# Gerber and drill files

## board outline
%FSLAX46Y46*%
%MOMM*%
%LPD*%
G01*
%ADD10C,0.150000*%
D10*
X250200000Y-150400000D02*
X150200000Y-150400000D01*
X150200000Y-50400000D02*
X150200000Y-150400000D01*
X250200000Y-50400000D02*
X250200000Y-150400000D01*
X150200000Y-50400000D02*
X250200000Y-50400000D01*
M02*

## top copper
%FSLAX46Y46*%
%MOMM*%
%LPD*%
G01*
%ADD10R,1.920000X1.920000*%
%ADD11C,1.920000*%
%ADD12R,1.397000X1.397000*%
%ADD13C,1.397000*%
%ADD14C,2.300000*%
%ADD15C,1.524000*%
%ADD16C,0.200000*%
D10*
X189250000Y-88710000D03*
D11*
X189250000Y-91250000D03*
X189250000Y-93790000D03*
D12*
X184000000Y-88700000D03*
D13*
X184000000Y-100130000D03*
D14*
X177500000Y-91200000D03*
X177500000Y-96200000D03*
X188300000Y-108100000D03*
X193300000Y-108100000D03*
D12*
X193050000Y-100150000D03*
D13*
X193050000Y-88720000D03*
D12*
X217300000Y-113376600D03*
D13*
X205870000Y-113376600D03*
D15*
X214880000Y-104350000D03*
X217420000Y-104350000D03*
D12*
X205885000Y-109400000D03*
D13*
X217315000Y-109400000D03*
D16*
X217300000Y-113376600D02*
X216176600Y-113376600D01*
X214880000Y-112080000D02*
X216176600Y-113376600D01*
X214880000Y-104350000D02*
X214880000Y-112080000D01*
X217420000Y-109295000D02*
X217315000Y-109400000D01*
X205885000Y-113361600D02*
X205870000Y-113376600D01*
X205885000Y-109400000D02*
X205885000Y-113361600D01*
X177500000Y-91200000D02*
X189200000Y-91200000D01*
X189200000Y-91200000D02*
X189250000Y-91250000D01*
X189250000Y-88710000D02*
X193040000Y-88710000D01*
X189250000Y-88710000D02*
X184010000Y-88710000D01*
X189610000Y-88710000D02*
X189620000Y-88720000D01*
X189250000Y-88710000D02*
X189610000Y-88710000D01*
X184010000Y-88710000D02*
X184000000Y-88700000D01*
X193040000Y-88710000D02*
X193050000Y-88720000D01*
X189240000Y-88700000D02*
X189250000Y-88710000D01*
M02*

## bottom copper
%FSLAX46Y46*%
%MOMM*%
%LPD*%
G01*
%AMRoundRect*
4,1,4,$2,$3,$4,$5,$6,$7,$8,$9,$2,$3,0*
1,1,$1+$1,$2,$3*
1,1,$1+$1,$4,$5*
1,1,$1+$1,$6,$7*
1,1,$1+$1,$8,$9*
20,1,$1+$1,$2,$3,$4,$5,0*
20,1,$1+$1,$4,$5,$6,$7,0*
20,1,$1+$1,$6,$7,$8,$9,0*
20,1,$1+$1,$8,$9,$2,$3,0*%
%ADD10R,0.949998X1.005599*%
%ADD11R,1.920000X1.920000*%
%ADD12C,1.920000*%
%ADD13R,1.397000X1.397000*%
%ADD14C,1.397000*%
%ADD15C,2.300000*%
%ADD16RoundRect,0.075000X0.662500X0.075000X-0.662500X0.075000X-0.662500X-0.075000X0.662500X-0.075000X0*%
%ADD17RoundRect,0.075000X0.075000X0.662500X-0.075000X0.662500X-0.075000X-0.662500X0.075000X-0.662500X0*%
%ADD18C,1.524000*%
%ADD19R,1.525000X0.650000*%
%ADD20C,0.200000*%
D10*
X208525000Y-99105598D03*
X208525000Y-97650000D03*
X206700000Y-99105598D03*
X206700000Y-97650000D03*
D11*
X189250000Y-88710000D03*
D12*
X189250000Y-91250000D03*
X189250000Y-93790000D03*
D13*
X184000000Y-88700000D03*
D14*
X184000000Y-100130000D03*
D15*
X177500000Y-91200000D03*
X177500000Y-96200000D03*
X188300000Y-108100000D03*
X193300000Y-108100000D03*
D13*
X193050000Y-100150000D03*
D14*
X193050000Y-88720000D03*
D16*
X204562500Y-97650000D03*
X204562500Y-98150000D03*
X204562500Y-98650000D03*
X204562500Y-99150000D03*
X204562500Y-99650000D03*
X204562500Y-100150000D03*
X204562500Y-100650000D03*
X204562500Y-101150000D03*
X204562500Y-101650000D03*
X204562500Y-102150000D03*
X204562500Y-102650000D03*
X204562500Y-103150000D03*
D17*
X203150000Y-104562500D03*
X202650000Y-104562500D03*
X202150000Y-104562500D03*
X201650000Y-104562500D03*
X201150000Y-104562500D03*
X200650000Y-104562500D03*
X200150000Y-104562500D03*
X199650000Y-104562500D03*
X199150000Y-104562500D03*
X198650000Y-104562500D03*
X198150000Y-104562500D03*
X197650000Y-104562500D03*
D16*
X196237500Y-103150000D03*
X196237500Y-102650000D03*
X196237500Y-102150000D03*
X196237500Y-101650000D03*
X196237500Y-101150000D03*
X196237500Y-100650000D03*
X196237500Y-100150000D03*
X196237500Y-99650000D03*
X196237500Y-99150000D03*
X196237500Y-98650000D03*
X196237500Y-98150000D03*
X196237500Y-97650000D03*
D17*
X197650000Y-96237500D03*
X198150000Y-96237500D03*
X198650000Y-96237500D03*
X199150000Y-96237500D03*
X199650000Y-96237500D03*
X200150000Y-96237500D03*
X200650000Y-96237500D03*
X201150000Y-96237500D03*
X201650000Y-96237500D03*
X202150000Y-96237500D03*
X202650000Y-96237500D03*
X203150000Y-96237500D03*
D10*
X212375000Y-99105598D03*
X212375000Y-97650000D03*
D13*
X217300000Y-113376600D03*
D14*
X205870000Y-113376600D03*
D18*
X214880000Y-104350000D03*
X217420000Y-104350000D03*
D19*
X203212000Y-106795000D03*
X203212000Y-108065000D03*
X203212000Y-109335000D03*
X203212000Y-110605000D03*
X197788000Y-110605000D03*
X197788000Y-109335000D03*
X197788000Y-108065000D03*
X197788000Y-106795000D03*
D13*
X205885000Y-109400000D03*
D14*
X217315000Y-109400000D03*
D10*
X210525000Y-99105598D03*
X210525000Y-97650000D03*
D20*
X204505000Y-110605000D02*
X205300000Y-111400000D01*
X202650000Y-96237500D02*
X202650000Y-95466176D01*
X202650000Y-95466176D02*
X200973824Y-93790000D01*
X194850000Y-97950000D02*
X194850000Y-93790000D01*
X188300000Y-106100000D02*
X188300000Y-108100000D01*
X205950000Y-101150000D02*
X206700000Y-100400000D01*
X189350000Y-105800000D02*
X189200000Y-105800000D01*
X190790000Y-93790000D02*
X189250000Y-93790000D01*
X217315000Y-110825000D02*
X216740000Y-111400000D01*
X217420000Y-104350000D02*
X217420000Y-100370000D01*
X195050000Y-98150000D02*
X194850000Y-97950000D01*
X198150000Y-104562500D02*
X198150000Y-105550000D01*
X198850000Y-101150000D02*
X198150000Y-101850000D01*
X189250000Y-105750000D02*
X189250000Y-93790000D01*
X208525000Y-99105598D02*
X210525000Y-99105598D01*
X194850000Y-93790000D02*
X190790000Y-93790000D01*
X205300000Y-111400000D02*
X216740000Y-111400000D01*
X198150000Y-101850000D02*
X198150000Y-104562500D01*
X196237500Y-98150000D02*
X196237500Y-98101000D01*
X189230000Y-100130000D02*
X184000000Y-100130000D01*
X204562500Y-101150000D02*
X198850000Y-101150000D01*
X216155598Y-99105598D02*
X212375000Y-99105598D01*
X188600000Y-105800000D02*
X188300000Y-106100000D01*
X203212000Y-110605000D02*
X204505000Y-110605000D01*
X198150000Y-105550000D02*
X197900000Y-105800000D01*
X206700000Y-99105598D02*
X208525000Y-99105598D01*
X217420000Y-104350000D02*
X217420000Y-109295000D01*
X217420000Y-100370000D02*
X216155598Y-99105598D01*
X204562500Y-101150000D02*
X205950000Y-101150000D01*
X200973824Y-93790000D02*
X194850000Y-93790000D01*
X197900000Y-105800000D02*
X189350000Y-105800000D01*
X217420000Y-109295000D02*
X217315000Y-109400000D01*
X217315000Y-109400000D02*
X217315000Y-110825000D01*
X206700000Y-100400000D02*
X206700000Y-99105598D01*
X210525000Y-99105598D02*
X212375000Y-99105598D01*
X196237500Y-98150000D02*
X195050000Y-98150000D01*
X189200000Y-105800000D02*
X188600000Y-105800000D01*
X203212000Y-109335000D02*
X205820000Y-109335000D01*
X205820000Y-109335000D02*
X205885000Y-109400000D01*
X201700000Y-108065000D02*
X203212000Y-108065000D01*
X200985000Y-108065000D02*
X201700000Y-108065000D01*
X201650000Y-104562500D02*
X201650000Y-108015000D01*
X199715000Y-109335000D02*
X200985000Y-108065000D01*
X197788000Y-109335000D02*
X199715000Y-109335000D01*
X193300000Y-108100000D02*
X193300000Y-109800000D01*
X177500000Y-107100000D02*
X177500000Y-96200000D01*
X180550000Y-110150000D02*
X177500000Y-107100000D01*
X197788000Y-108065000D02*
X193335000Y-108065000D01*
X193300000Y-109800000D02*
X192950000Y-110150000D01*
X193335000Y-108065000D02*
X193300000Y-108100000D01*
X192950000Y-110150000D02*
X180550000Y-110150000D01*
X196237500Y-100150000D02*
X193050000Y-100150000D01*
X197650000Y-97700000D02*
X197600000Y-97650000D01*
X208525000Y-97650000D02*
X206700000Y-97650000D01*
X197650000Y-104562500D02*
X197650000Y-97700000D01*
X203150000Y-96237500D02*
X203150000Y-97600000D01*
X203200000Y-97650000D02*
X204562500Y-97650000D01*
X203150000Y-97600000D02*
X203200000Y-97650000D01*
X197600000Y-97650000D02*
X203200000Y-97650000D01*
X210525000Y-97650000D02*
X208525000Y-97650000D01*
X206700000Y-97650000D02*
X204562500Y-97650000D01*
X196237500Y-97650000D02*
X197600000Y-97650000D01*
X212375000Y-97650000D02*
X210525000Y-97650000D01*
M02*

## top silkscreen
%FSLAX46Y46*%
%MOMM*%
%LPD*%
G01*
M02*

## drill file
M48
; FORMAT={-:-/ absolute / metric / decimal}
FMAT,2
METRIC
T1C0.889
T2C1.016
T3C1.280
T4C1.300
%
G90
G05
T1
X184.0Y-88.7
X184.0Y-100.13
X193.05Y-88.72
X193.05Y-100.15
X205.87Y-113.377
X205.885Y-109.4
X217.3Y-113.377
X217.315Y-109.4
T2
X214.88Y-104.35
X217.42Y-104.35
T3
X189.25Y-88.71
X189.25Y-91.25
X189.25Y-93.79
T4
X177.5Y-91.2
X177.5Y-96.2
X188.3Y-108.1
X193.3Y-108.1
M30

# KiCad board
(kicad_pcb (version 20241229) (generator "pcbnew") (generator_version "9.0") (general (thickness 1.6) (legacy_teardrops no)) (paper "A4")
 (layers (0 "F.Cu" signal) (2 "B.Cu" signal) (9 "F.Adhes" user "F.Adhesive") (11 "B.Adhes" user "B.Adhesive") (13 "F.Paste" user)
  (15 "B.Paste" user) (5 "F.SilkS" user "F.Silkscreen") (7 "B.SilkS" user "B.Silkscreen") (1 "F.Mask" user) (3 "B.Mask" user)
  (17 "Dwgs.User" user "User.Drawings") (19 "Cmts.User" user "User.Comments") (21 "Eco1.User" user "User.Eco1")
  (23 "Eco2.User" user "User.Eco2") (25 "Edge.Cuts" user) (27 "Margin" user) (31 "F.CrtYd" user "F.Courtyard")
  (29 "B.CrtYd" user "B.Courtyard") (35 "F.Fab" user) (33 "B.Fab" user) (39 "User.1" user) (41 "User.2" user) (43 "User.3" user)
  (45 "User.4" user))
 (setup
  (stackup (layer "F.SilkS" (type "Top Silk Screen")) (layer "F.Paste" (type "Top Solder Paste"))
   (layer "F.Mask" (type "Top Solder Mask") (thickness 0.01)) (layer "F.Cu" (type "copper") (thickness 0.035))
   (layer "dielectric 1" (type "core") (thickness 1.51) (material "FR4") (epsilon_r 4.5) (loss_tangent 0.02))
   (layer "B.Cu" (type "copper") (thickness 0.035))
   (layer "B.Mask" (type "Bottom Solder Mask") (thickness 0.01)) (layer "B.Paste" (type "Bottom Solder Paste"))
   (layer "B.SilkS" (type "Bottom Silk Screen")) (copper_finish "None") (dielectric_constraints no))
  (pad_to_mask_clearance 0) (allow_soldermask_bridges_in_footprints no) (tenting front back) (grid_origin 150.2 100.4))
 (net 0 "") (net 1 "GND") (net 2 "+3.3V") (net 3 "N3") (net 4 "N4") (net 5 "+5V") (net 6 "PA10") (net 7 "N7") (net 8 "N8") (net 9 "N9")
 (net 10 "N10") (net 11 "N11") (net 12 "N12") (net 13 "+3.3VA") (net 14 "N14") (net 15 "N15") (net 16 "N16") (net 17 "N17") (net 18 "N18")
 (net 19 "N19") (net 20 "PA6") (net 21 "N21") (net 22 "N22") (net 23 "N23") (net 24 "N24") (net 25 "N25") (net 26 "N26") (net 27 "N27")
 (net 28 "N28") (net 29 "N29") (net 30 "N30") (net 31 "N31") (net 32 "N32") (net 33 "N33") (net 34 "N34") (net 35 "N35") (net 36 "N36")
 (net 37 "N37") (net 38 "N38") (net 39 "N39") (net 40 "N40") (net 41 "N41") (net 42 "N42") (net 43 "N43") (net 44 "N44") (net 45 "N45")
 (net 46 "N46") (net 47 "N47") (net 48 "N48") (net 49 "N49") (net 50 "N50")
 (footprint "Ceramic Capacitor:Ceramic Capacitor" (layer "B.Cu") (at 208.525 98.377799 90)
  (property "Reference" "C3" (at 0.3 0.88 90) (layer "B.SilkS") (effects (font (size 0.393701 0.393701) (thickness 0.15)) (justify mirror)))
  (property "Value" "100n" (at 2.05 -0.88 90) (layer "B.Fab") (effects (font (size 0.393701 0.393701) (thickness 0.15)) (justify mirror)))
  (pad "1" smd rect (at -0.727799 0 90) (size 1.005599 0.949998) (layers "B.Cu" "B.Mask" "B.Paste") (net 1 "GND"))
  (pad "2" smd rect (at 0.727799 0 90) (size 1.005599 0.949998) (layers "B.Cu" "B.Mask" "B.Paste") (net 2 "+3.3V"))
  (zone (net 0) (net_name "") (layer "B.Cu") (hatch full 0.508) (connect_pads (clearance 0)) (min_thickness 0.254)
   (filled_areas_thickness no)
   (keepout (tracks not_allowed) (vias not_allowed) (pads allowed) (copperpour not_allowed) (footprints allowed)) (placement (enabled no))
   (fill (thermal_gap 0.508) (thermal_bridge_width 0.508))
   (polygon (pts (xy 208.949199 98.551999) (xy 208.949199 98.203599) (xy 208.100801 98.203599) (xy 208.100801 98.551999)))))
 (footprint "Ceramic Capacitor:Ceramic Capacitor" (layer "B.Cu") (at 206.7 98.377799 90)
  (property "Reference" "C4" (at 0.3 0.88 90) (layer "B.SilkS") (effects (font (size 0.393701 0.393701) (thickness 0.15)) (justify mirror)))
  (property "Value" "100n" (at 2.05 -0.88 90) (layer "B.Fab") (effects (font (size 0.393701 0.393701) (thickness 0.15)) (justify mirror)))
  (pad "1" smd rect (at -0.727799 0 90) (size 1.005599 0.949998) (layers "B.Cu" "B.Mask" "B.Paste") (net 1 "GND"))
  (pad "2" smd rect (at 0.727799 0 90) (size 1.005599 0.949998) (layers "B.Cu" "B.Mask" "B.Paste") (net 2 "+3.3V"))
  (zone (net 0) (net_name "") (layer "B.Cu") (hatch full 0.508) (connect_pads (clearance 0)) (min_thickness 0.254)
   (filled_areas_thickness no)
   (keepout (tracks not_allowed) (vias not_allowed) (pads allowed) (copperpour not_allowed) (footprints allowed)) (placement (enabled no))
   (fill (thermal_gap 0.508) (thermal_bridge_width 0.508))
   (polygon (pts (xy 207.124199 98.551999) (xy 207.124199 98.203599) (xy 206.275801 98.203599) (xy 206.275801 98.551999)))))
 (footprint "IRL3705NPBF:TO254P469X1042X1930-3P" (layer "B.Cu") (at 189.25 88.71 -90)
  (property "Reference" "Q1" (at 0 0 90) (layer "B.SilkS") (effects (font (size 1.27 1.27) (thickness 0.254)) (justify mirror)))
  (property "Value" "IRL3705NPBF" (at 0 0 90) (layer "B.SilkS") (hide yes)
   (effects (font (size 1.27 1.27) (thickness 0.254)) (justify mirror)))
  (pad "1" thru_hole rect (at 0 0 270) (size 1.92 1.92) (drill 1.28) (layers "*.Cu" "*.Mask") (remove_unused_layers no) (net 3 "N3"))
  (pad "2" thru_hole circle (at 2.54 0 270) (size 1.92 1.92) (drill 1.28) (layers "*.Cu" "*.Mask") (remove_unused_layers no) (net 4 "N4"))
  (pad "3" thru_hole circle (at 5.08 0 270) (size 1.92 1.92) (drill 1.28) (layers "*.Cu" "*.Mask") (remove_unused_layers no) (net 1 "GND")))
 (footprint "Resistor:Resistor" (layer "B.Cu") (at 184 88.7 -90)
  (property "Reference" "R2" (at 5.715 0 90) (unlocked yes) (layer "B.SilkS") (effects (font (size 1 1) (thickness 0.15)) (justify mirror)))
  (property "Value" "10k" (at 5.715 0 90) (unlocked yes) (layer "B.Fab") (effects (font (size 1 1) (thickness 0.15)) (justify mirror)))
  (pad "1" thru_hole rect (at 0 0 270) (size 1.397 1.397) (drill 0.889) (layers "*.Cu" "*.Mask") (remove_unused_layers no) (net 3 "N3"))
  (pad "2" thru_hole circle (at 11.43 0 270) (size 1.397 1.397) (drill 0.889) (layers "*.Cu" "*.Mask") (remove_unused_layers no)
   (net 1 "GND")))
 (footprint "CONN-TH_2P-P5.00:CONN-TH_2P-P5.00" (layer "B.Cu") (at 181.75 88.7 -90)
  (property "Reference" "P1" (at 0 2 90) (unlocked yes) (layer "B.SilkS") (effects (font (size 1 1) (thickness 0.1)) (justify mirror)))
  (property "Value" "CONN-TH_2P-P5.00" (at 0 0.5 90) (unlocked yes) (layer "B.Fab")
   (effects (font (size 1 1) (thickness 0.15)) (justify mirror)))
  (pad "1" thru_hole circle (at 2.5 4.25 270) (size 2.3 2.3) (drill 1.3) (layers "*.Cu" "*.Mask") (remove_unused_layers no) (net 4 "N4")
   (solder_mask_margin 0.07))
  (pad "2" thru_hole circle (at 7.5 4.25 270) (size 2.3 2.3) (drill 1.3) (layers "*.Cu" "*.Mask") (remove_unused_layers no) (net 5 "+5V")
   (solder_mask_margin 0.07)))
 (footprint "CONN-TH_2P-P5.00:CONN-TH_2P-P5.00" (layer "B.Cu") (at 185.8 103.85)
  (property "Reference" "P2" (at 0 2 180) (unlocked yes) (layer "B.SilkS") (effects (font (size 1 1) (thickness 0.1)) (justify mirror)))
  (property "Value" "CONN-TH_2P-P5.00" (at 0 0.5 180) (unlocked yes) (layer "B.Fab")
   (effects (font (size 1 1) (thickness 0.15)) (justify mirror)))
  (pad "1" thru_hole circle (at 2.5 4.25) (size 2.3 2.3) (drill 1.3) (layers "*.Cu" "*.Mask") (remove_unused_layers no) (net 1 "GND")
   (solder_mask_margin 0.07))
  (pad "2" thru_hole circle (at 7.5 4.25) (size 2.3 2.3) (drill 1.3) (layers "*.Cu" "*.Mask") (remove_unused_layers no) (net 5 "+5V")
   (solder_mask_margin 0.07)))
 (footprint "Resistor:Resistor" (layer "B.Cu") (at 193.05 100.15 90)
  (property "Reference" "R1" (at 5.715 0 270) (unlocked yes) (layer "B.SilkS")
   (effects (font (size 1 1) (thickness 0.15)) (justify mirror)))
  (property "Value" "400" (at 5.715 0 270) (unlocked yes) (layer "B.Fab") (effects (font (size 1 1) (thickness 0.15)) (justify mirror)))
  (pad "1" thru_hole rect (at 0 0 90) (size 1.397 1.397) (drill 0.889) (layers "*.Cu" "*.Mask") (remove_unused_layers no) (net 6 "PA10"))
  (pad "2" thru_hole circle (at 11.43 0 90) (size 1.397 1.397) (drill 0.889) (layers "*.Cu" "*.Mask") (remove_unused_layers no) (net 3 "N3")))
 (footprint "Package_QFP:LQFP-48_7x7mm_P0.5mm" (layer "B.Cu") (at 200.4 100.4 180)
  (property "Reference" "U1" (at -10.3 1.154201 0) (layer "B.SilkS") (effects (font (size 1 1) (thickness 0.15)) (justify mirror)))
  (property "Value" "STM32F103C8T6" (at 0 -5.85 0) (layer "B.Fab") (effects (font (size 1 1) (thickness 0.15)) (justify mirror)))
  (pad "1" smd roundrect (at -4.1625 2.75 180) (size 1.475 0.3) (layers "B.Cu" "B.Mask" "B.Paste") (roundrect_rratio 0.25) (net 2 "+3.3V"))
  (pad "2" smd roundrect (at -4.1625 2.25 180) (size 1.475 0.3) (layers "B.Cu" "B.Mask" "B.Paste") (roundrect_rratio 0.25) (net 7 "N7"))
  (pad "3" smd roundrect (at -4.1625 1.75 180) (size 1.475 0.3) (layers "B.Cu" "B.Mask" "B.Paste") (roundrect_rratio 0.25) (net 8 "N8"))
  (pad "4" smd roundrect (at -4.1625 1.25 180) (size 1.475 0.3) (layers "B.Cu" "B.Mask" "B.Paste") (roundrect_rratio 0.25) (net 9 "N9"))
  (pad "5" smd roundrect (at -4.1625 0.75 180) (size 1.475 0.3) (layers "B.Cu" "B.Mask" "B.Paste") (roundrect_rratio 0.25) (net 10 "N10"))
  (pad "6" smd roundrect (at -4.1625 0.25 180) (size 1.475 0.3) (layers "B.Cu" "B.Mask" "B.Paste") (roundrect_rratio 0.25) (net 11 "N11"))
  (pad "7" smd roundrect (at -4.1625 -0.25 180) (size 1.475 0.3) (layers "B.Cu" "B.Mask" "B.Paste") (roundrect_rratio 0.25) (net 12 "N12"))
  (pad "8" smd roundrect (at -4.1625 -0.75 180) (size 1.475 0.3) (layers "B.Cu" "B.Mask" "B.Paste") (roundrect_rratio 0.25) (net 1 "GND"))
  (pad "9" smd roundrect (at -4.1625 -1.25 180) (size 1.475 0.3) (layers "B.Cu" "B.Mask" "B.Paste") (roundrect_rratio 0.25)
   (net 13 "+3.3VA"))
  (pad "10" smd roundrect (at -4.1625 -1.75 180) (size 1.475 0.3) (layers "B.Cu" "B.Mask" "B.Paste") (roundrect_rratio 0.25) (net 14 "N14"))
  (pad "11" smd roundrect (at -4.1625 -2.25 180) (size 1.475 0.3) (layers "B.Cu" "B.Mask" "B.Paste") (roundrect_rratio 0.25) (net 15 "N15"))
  (pad "12" smd roundrect (at -4.1625 -2.75 180) (size 1.475 0.3) (layers "B.Cu" "B.Mask" "B.Paste") (roundrect_rratio 0.25) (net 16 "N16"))
  (pad "13" smd roundrect (at -2.75 -4.1625 180) (size 0.3 1.475) (layers "B.Cu" "B.Mask" "B.Paste") (roundrect_rratio 0.25) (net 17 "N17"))
  (pad "14" smd roundrect (at -2.25 -4.1625 180) (size 0.3 1.475) (layers "B.Cu" "B.Mask" "B.Paste") (roundrect_rratio 0.25) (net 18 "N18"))
  (pad "15" smd roundrect (at -1.75 -4.1625 180) (size 0.3 1.475) (layers "B.Cu" "B.Mask" "B.Paste") (roundrect_rratio 0.25) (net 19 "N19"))
  (pad "16" smd roundrect (at -1.25 -4.1625 180) (size 0.3 1.475) (layers "B.Cu" "B.Mask" "B.Paste") (roundrect_rratio 0.25) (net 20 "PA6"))
  (pad "17" smd roundrect (at -0.75 -4.1625 180) (size 0.3 1.475) (layers "B.Cu" "B.Mask" "B.Paste") (roundrect_rratio 0.25) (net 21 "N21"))
  (pad "18" smd roundrect (at -0.25 -4.1625 180) (size 0.3 1.475) (layers "B.Cu" "B.Mask" "B.Paste") (roundrect_rratio 0.25) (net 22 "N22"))
  (pad "19" smd roundrect (at 0.25 -4.1625 180) (size 0.3 1.475) (layers "B.Cu" "B.Mask" "B.Paste") (roundrect_rratio 0.25) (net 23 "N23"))
  (pad "20" smd roundrect (at 0.75 -4.1625 180) (size 0.3 1.475) (layers "B.Cu" "B.Mask" "B.Paste") (roundrect_rratio 0.25) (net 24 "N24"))
  (pad "21" smd roundrect (at 1.25 -4.1625 180) (size 0.3 1.475) (layers "B.Cu" "B.Mask" "B.Paste") (roundrect_rratio 0.25) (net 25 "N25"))
  (pad "22" smd roundrect (at 1.75 -4.1625 180) (size 0.3 1.475) (layers "B.Cu" "B.Mask" "B.Paste") (roundrect_rratio 0.25) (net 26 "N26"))
  (pad "23" smd roundrect (at 2.25 -4.1625 180) (size 0.3 1.475) (layers "B.Cu" "B.Mask" "B.Paste") (roundrect_rratio 0.25) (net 1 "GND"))
  (pad "24" smd roundrect (at 2.75 -4.1625 180) (size 0.3 1.475) (layers "B.Cu" "B.Mask" "B.Paste") (roundrect_rratio 0.25) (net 2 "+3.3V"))
  (pad "25" smd roundrect (at 4.1625 -2.75 180) (size 1.475 0.3) (layers "B.Cu" "B.Mask" "B.Paste") (roundrect_rratio 0.25) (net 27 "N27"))
  (pad "26" smd roundrect (at 4.1625 -2.25 180) (size 1.475 0.3) (layers "B.Cu" "B.Mask" "B.Paste") (roundrect_rratio 0.25) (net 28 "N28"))
  (pad "27" smd roundrect (at 4.1625 -1.75 180) (size 1.475 0.3) (layers "B.Cu" "B.Mask" "B.Paste") (roundrect_rratio 0.25) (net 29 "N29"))
  (pad "28" smd roundrect (at 4.1625 -1.25 180) (size 1.475 0.3) (layers "B.Cu" "B.Mask" "B.Paste") (roundrect_rratio 0.25) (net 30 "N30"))
  (pad "29" smd roundrect (at 4.1625 -0.75 180) (size 1.475 0.3) (layers "B.Cu" "B.Mask" "B.Paste") (roundrect_rratio 0.25) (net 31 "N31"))
  (pad "30" smd roundrect (at 4.1625 -0.25 180) (size 1.475 0.3) (layers "B.Cu" "B.Mask" "B.Paste") (roundrect_rratio 0.25) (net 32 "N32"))
  (pad "31" smd roundrect (at 4.1625 0.25 180) (size 1.475 0.3) (layers "B.Cu" "B.Mask" "B.Paste") (roundrect_rratio 0.25) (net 6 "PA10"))
  (pad "32" smd roundrect (at 4.1625 0.75 180) (size 1.475 0.3) (layers "B.Cu" "B.Mask" "B.Paste") (roundrect_rratio 0.25) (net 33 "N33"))
  (pad "33" smd roundrect (at 4.1625 1.25 180) (size 1.475 0.3) (layers "B.Cu" "B.Mask" "B.Paste") (roundrect_rratio 0.25) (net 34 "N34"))
  (pad "34" smd roundrect (at 4.1625 1.75 180) (size 1.475 0.3) (layers "B.Cu" "B.Mask" "B.Paste") (roundrect_rratio 0.25) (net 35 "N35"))
  (pad "35" smd roundrect (at 4.1625 2.25 180) (size 1.475 0.3) (layers "B.Cu" "B.Mask" "B.Paste") (roundrect_rratio 0.25) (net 1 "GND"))
  (pad "36" smd roundrect (at 4.1625 2.75 180) (size 1.475 0.3) (layers "B.Cu" "B.Mask" "B.Paste") (roundrect_rratio 0.25) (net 2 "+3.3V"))
  (pad "37" smd roundrect (at 2.75 4.1625 180) (size 0.3 1.475) (layers "B.Cu" "B.Mask" "B.Paste") (roundrect_rratio 0.25) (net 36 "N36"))
  (pad "38" smd roundrect (at 2.25 4.1625 180) (size 0.3 1.475) (layers "B.Cu" "B.Mask" "B.Paste") (roundrect_rratio 0.25) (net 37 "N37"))
  (pad "39" smd roundrect (at 1.75 4.1625 180) (size 0.3 1.475) (layers "B.Cu" "B.Mask" "B.Paste") (roundrect_rratio 0.25) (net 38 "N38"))
  (pad "40" smd roundrect (at 1.25 4.1625 180) (size 0.3 1.475) (layers "B.Cu" "B.Mask" "B.Paste") (roundrect_rratio 0.25) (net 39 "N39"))
  (pad "41" smd roundrect (at 0.75 4.1625 180) (size 0.3 1.475) (layers "B.Cu" "B.Mask" "B.Paste") (roundrect_rratio 0.25) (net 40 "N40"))
  (pad "42" smd roundrect (at 0.25 4.1625 180) (size 0.3 1.475) (layers "B.Cu" "B.Mask" "B.Paste") (roundrect_rratio 0.25) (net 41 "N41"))
  (pad "43" smd roundrect (at -0.25 4.1625 180) (size 0.3 1.475) (layers "B.Cu" "B.Mask" "B.Paste") (roundrect_rratio 0.25) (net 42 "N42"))
  (pad "44" smd roundrect (at -0.75 4.1625 180) (size 0.3 1.475) (layers "B.Cu" "B.Mask" "B.Paste") (roundrect_rratio 0.25) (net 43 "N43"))
  (pad "45" smd roundrect (at -1.25 4.1625 180) (size 0.3 1.475) (layers "B.Cu" "B.Mask" "B.Paste") (roundrect_rratio 0.25) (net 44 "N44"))
  (pad "46" smd roundrect (at -1.75 4.1625 180) (size 0.3 1.475) (layers "B.Cu" "B.Mask" "B.Paste") (roundrect_rratio 0.25) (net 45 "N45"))
  (pad "47" smd roundrect (at -2.25 4.1625 180) (size 0.3 1.475) (layers "B.Cu" "B.Mask" "B.Paste") (roundrect_rratio 0.25) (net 1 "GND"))
  (pad "48" smd roundrect (at -2.75 4.1625 180) (size 0.3 1.475) (layers "B.Cu" "B.Mask" "B.Paste") (roundrect_rratio 0.25) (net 2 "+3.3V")))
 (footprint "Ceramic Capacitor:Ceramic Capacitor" (layer "B.Cu") (at 212.375 98.377799 90)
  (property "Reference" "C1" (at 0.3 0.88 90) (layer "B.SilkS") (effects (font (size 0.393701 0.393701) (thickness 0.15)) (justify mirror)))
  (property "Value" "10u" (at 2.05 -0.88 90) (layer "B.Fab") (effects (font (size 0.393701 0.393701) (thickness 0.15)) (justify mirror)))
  (pad "1" smd rect (at -0.727799 0 90) (size 1.005599 0.949998) (layers "B.Cu" "B.Mask" "B.Paste") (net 1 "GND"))
  (pad "2" smd rect (at 0.727799 0 90) (size 1.005599 0.949998) (layers "B.Cu" "B.Mask" "B.Paste") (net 2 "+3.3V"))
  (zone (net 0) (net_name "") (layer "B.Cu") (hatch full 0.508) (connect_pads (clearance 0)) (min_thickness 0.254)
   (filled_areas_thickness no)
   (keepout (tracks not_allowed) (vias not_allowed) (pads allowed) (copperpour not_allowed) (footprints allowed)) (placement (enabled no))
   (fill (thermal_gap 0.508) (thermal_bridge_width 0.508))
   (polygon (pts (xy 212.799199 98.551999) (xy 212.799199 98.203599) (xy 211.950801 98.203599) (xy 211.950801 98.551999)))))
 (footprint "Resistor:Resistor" (layer "B.Cu") (at 217.3 113.3766 180)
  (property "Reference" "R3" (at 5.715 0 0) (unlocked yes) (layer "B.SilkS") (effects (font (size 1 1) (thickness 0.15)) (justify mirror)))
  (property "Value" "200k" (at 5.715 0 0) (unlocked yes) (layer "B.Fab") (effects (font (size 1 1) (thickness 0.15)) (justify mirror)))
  (pad "1" thru_hole rect (at 0 0 180) (size 1.397 1.397) (drill 0.889) (layers "*.Cu" "*.Mask") (remove_unused_layers no) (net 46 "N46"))
  (pad "2" thru_hole circle (at 11.43 0 180) (size 1.397 1.397) (drill 0.889) (layers "*.Cu" "*.Mask") (remove_unused_layers no)
   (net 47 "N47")))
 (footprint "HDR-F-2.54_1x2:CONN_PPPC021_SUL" (layer "B.Cu") (at 214.88 104.35 180)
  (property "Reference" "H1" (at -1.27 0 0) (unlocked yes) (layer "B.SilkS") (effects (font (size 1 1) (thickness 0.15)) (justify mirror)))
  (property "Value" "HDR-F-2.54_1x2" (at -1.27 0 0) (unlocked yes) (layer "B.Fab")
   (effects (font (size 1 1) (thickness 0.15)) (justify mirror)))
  (pad "1" thru_hole circle (at 0 0 180) (size 1.524 1.524) (drill 1.016) (layers "*.Cu" "*.Mask") (remove_unused_layers no) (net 46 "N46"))
  (pad "2" thru_hole circle (at -2.54 0 180) (size 1.524 1.524) (drill 1.016) (layers "*.Cu" "*.Mask") (remove_unused_layers no)
   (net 1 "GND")))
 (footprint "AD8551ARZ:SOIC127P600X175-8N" (layer "B.Cu") (at 200.5 108.7 180)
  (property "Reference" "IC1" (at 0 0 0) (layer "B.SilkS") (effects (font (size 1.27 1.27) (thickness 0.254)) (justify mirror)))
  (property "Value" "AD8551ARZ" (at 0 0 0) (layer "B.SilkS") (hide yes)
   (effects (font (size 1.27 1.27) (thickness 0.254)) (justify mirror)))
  (pad "1" smd rect (at -2.712 1.905 90) (size 0.65 1.525) (layers "B.Cu" "B.Mask" "B.Paste") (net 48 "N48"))
  (pad "2" smd rect (at -2.712 0.635 90) (size 0.65 1.525) (layers "B.Cu" "B.Mask" "B.Paste") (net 20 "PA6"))
  (pad "3" smd rect (at -2.712 -0.635 90) (size 0.65 1.525) (layers "B.Cu" "B.Mask" "B.Paste") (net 47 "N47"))
  (pad "4" smd rect (at -2.712 -1.905 90) (size 0.65 1.525) (layers "B.Cu" "B.Mask" "B.Paste") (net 1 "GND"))
  (pad "5" smd rect (at 2.712 -1.905 90) (size 0.65 1.525) (layers "B.Cu" "B.Mask" "B.Paste") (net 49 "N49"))
  (pad "6" smd rect (at 2.712 -0.635 90) (size 0.65 1.525) (layers "B.Cu" "B.Mask" "B.Paste") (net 20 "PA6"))
  (pad "7" smd rect (at 2.712 0.635 90) (size 0.65 1.525) (layers "B.Cu" "B.Mask" "B.Paste") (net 5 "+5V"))
  (pad "8" smd rect (at 2.712 1.905 90) (size 0.65 1.525) (layers "B.Cu" "B.Mask" "B.Paste") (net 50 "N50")))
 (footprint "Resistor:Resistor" (layer "B.Cu") (at 205.885 109.4)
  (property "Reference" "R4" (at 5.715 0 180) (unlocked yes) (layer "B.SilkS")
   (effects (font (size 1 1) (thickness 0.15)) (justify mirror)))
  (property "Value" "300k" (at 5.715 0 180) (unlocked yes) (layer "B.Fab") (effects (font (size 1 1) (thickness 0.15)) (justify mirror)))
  (pad "1" thru_hole rect (at 0 0) (size 1.397 1.397) (drill 0.889) (layers "*.Cu" "*.Mask") (remove_unused_layers no) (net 47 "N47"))
  (pad "2" thru_hole circle (at 11.43 0) (size 1.397 1.397) (drill 0.889) (layers "*.Cu" "*.Mask") (remove_unused_layers no) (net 1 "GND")))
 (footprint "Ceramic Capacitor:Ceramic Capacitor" (layer "B.Cu") (at 210.525 98.377799 90)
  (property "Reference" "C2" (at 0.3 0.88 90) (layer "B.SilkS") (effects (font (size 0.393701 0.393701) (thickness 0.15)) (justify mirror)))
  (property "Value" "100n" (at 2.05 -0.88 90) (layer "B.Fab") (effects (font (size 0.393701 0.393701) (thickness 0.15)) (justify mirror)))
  (pad "1" smd rect (at -0.727799 0 90) (size 1.005599 0.949998) (layers "B.Cu" "B.Mask" "B.Paste") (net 1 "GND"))
  (pad "2" smd rect (at 0.727799 0 90) (size 1.005599 0.949998) (layers "B.Cu" "B.Mask" "B.Paste") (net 2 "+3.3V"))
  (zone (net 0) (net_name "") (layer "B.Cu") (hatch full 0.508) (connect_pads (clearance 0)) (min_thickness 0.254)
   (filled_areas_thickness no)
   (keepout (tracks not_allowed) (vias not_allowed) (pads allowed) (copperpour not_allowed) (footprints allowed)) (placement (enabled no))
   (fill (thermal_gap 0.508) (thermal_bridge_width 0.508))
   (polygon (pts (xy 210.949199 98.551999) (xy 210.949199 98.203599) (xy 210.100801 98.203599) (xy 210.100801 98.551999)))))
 (gr_line (start 250.2 150.4) (end 150.2 150.4) (stroke (width 0.15) (type default)) (layer "Edge.Cuts"))
 (gr_line (start 150.2 50.4) (end 150.2 150.4) (stroke (width 0.15) (type default)) (layer "Edge.Cuts"))
 (gr_line (start 250.2 50.4) (end 250.2 150.4) (stroke (width 0.15) (type default)) (layer "Edge.Cuts"))
 (gr_line (start 150.2 50.4) (end 250.2 50.4) (stroke (width 0.15) (type default)) (layer "Edge.Cuts"))
 (segment (start 217.3 113.3766) (end 216.1766 113.3766) (width 0.2) (layer "F.Cu") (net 46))
 (segment (start 214.88 112.08) (end 216.1766 113.3766) (width 0.2) (layer "F.Cu") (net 46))
 (segment (start 214.88 104.35) (end 214.88 112.08) (width 0.2) (layer "F.Cu") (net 46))
 (segment (start 217.42 109.295) (end 217.315 109.4) (width 0.2) (layer "F.Cu") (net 1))
 (segment (start 204.505 110.605) (end 205.3 111.4) (width 0.2) (layer "B.Cu") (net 1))
 (segment (start 202.65 96.2375) (end 202.65 95.466176) (width 0.2) (layer "B.Cu") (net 1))
 (segment (start 202.65 95.466176) (end 200.973824 93.79) (width 0.2) (layer "B.Cu") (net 1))
 (segment (start 194.85 97.95) (end 194.85 93.79) (width 0.2) (layer "B.Cu") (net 1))
 (segment (start 188.3 106.1) (end 188.3 108.1) (width 0.2) (layer "B.Cu") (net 1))
 (segment (start 205.95 101.15) (end 206.7 100.4) (width 0.2) (layer "B.Cu") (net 1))
 (segment (start 189.35 105.8) (end 189.2 105.8) (width 0.2) (layer "B.Cu") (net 1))
 (segment (start 190.79 93.79) (end 189.25 93.79) (width 0.2) (layer "B.Cu") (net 1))
 (segment (start 217.315 110.825) (end 216.74 111.4) (width 0.2) (layer "B.Cu") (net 1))
 (segment (start 217.42 104.35) (end 217.42 100.37) (width 0.2) (layer "B.Cu") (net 1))
 (segment (start 195.05 98.15) (end 194.85 97.95) (width 0.2) (layer "B.Cu") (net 1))
 (segment (start 198.15 104.5625) (end 198.15 105.55) (width 0.2) (layer "B.Cu") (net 1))
 (segment (start 198.85 101.15) (end 198.15 101.85) (width 0.2) (layer "B.Cu") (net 1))
 (segment (start 189.25 105.75) (end 189.25 93.79) (width 0.2) (layer "B.Cu") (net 1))
 (segment (start 208.525 99.105598) (end 210.525 99.105598) (width 0.2) (layer "B.Cu") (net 1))
 (segment (start 194.85 93.79) (end 190.79 93.79) (width 0.2) (layer "B.Cu") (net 1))
 (segment (start 205.3 111.4) (end 216.74 111.4) (width 0.2) (layer "B.Cu") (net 1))
 (segment (start 198.15 101.85) (end 198.15 104.5625) (width 0.2) (layer "B.Cu") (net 1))
 (segment (start 196.2375 98.15) (end 196.2375 98.101) (width 0.2) (layer "B.Cu") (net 1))
 (segment (start 189.23 100.13) (end 184 100.13) (width 0.2) (layer "B.Cu") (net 1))
 (segment (start 204.5625 101.15) (end 198.85 101.15) (width 0.2) (layer "B.Cu") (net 1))
 (segment (start 216.155598 99.105598) (end 212.375 99.105598) (width 0.2) (layer "B.Cu") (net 1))
 (segment (start 188.6 105.8) (end 188.3 106.1) (width 0.2) (layer "B.Cu") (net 1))
 (segment (start 203.212 110.605) (end 204.505 110.605) (width 0.2) (layer "B.Cu") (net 1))
 (segment (start 198.15 105.55) (end 197.9 105.8) (width 0.2) (layer "B.Cu") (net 1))
 (segment (start 206.7 99.105598) (end 208.525 99.105598) (width 0.2) (layer "B.Cu") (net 1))
 (segment (start 217.42 104.35) (end 217.42 109.295) (width 0.2) (layer "B.Cu") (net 1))
 (segment (start 217.42 100.37) (end 216.155598 99.105598) (width 0.2) (layer "B.Cu") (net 1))
 (segment (start 204.5625 101.15) (end 205.95 101.15) (width 0.2) (layer "B.Cu") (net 1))
 (segment (start 200.973824 93.79) (end 194.85 93.79) (width 0.2) (layer "B.Cu") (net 1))
 (segment (start 197.9 105.8) (end 189.35 105.8) (width 0.2) (layer "B.Cu") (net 1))
 (segment (start 217.42 109.295) (end 217.315 109.4) (width 0.2) (layer "B.Cu") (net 1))
 (segment (start 217.315 109.4) (end 217.315 110.825) (width 0.2) (layer "B.Cu") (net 1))
 (segment (start 206.7 100.4) (end 206.7 99.105598) (width 0.2) (layer "B.Cu") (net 1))
 (segment (start 210.525 99.105598) (end 212.375 99.105598) (width 0.2) (layer "B.Cu") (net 1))
 (segment (start 196.2375 98.15) (end 195.05 98.15) (width 0.2) (layer "B.Cu") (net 1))
 (segment (start 189.2 105.8) (end 188.6 105.8) (width 0.2) (layer "B.Cu") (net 1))
 (segment (start 205.885 113.3616) (end 205.87 113.3766) (width 0.2) (layer "F.Cu") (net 47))
 (segment (start 205.885 109.4) (end 205.885 113.3616) (width 0.2) (layer "F.Cu") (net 47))
 (segment (start 203.212 109.335) (end 205.82 109.335) (width 0.2) (layer "B.Cu") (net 47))
 (segment (start 205.82 109.335) (end 205.885 109.4) (width 0.2) (layer "B.Cu") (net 47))
 (segment (start 201.7 108.065) (end 203.212 108.065) (width 0.2) (layer "B.Cu") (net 20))
 (segment (start 200.985 108.065) (end 201.7 108.065) (width 0.2) (layer "B.Cu") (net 20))
 (segment (start 201.65 104.5625) (end 201.65 108.015) (width 0.2) (layer "B.Cu") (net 20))
 (segment (start 199.715 109.335) (end 200.985 108.065) (width 0.2) (layer "B.Cu") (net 20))
 (segment (start 197.788 109.335) (end 199.715 109.335) (width 0.2) (layer "B.Cu") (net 20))
 (segment (start 193.3 108.1) (end 193.3 109.8) (width 0.2) (layer "B.Cu") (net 5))
 (segment (start 177.5 107.1) (end 177.5 96.2) (width 0.2) (layer "B.Cu") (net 5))
 (segment (start 180.55 110.15) (end 177.5 107.1) (width 0.2) (layer "B.Cu") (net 5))
 (segment (start 197.788 108.065) (end 193.335 108.065) (width 0.2) (layer "B.Cu") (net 5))
 (segment (start 193.3 109.8) (end 192.95 110.15) (width 0.2) (layer "B.Cu") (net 5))
 (segment (start 193.335 108.065) (end 193.3 108.1) (width 0.2) (layer "B.Cu") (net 5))
 (segment (start 192.95 110.15) (end 180.55 110.15) (width 0.2) (layer "B.Cu") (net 5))
 (segment (start 177.5 91.2) (end 189.2 91.2) (width 0.2) (layer "F.Cu") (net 4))
 (segment (start 189.2 91.2) (end 189.25 91.25) (width 0.2) (layer "F.Cu") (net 4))
 (segment (start 189.25 88.71) (end 193.04 88.71) (width 0.2) (layer "F.Cu") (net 3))
 (segment (start 189.25 88.71) (end 184.01 88.71) (width 0.2) (layer "F.Cu") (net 3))
 (segment (start 189.61 88.71) (end 189.62 88.72) (width 0.2) (layer "F.Cu") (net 3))
 (segment (start 189.25 88.71) (end 189.61 88.71) (width 0.2) (layer "F.Cu") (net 3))
 (segment (start 184.01 88.71) (end 184 88.7) (width 0.2) (layer "F.Cu") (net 3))
 (segment (start 193.04 88.71) (end 193.05 88.72) (width 0.2) (layer "F.Cu") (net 3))
 (segment (start 189.24 88.7) (end 189.25 88.71) (width 0.2) (layer "F.Cu") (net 3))
 (segment (start 196.2375 100.15) (end 193.05 100.15) (width 0.2) (layer "B.Cu") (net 6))
 (segment (start 197.65 97.7) (end 197.6 97.65) (width 0.2) (layer "B.Cu") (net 2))
 (segment (start 208.525 97.65) (end 206.7 97.65) (width 0.2) (layer "B.Cu") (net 2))
 (segment (start 197.65 104.5625) (end 197.65 97.7) (width 0.2) (layer "B.Cu") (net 2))
 (segment (start 203.15 96.2375) (end 203.15 97.6) (width 0.2) (layer "B.Cu") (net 2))
 (segment (start 203.2 97.65) (end 204.5625 97.65) (width 0.2) (layer "B.Cu") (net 2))
 (segment (start 203.15 97.6) (end 203.2 97.65) (width 0.2) (layer "B.Cu") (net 2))
 (segment (start 197.6 97.65) (end 203.2 97.65) (width 0.2) (layer "B.Cu") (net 2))
 (segment (start 210.525 97.65) (end 208.525 97.65) (width 0.2) (layer "B.Cu") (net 2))
 (segment (start 206.7 97.65) (end 204.5625 97.65) (width 0.2) (layer "B.Cu") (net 2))
 (segment (start 196.2375 97.65) (end 197.6 97.65) (width 0.2) (layer "B.Cu") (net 2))
 (segment (start 212.375 97.65) (end 210.525 97.65) (width 0.2) (layer "B.Cu") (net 2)))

